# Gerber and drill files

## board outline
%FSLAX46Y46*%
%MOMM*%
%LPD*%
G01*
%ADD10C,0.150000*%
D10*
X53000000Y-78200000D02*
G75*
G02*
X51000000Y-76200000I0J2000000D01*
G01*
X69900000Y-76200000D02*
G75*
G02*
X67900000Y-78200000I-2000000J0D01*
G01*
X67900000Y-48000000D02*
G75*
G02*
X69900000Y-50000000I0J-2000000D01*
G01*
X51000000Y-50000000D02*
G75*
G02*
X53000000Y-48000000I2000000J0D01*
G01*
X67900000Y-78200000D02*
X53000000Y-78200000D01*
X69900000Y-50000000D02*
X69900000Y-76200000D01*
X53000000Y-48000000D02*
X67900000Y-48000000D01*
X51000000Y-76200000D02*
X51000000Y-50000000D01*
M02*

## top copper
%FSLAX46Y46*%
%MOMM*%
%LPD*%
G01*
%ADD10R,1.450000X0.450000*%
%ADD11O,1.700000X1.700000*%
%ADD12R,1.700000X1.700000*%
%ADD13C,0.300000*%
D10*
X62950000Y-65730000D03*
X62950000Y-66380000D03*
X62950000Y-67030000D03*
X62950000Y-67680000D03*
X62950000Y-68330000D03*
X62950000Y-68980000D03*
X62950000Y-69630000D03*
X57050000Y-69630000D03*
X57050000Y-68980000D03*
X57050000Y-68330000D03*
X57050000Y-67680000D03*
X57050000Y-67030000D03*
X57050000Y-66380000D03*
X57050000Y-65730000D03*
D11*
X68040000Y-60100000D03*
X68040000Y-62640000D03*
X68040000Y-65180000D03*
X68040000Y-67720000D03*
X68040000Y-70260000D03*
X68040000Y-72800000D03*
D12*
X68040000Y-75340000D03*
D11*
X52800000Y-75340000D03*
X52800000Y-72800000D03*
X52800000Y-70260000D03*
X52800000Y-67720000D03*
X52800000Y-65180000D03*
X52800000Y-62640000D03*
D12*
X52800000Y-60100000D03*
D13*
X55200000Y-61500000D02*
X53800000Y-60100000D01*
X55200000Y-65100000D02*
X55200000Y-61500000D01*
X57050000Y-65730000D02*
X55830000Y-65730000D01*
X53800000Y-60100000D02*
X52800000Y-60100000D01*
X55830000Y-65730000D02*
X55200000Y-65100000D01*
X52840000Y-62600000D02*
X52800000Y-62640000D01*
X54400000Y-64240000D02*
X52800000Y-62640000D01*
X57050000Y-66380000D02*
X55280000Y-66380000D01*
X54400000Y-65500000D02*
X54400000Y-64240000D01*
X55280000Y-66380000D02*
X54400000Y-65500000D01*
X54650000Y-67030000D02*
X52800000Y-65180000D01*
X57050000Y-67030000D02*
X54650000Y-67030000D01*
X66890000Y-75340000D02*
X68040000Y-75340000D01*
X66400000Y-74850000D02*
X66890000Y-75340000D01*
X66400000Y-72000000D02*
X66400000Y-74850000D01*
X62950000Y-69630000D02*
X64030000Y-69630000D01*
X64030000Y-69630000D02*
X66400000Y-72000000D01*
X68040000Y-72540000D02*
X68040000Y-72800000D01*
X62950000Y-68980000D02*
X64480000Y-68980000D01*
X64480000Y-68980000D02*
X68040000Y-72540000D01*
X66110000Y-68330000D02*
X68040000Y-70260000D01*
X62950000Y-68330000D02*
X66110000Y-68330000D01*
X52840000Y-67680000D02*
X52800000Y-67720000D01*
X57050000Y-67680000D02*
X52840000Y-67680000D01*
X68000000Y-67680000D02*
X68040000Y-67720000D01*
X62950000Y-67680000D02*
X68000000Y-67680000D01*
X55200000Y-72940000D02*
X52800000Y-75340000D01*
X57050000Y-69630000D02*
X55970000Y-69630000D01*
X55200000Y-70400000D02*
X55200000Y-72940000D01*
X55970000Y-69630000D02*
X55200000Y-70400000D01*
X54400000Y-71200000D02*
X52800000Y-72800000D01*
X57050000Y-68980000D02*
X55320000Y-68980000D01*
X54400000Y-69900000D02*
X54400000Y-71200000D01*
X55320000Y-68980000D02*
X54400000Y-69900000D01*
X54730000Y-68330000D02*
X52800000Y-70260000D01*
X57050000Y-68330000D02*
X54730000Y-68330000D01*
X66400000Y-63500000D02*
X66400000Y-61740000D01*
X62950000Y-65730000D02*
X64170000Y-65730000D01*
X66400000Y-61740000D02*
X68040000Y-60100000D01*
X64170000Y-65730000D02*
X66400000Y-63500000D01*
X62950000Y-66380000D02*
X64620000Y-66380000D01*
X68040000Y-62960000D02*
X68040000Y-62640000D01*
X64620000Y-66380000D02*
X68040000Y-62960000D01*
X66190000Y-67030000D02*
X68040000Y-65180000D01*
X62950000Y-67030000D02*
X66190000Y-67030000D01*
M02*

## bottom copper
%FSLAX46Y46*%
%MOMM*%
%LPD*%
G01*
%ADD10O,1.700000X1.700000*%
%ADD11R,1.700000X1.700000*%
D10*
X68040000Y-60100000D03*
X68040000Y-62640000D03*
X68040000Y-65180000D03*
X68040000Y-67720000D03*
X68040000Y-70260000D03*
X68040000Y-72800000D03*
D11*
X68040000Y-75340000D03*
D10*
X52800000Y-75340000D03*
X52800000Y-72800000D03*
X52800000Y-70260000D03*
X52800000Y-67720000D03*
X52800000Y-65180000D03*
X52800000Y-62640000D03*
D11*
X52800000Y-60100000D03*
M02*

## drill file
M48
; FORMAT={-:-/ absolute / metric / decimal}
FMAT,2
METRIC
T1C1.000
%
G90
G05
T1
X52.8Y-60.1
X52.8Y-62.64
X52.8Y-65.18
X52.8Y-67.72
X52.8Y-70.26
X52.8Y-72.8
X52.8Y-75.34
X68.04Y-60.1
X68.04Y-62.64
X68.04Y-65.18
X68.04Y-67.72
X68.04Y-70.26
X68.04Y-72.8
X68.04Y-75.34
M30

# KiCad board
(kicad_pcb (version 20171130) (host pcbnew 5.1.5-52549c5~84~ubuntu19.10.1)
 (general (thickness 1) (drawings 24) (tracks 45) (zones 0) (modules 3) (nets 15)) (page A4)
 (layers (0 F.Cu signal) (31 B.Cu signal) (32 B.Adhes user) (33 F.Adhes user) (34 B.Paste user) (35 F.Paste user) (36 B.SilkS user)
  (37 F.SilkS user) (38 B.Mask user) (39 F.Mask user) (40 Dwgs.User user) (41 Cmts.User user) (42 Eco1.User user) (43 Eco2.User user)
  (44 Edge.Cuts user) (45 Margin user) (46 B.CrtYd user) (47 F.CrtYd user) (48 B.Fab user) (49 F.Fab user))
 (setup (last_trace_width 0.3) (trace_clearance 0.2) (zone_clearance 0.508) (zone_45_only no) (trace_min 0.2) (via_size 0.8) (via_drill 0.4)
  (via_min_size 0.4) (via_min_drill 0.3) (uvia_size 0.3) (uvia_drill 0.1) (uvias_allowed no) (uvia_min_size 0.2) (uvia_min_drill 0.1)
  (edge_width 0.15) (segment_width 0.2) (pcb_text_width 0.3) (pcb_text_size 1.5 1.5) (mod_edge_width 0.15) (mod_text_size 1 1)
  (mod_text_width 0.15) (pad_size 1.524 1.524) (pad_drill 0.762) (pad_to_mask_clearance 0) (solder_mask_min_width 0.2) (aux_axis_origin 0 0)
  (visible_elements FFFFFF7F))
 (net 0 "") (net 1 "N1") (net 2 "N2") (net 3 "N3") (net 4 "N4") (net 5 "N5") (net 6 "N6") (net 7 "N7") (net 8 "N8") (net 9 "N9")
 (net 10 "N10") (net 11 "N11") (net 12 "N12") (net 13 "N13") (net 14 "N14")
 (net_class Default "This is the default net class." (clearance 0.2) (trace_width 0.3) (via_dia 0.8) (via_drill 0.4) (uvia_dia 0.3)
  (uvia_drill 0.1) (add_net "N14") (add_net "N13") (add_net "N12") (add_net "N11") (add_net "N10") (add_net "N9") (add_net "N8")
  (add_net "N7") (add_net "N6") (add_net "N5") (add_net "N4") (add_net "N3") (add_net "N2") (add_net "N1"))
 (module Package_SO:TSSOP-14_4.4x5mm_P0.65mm (layer F.Cu) (at 60 67.68)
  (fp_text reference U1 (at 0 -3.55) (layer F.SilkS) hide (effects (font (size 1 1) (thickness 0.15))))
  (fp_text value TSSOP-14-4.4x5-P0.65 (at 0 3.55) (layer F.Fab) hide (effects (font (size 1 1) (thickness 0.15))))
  (pad 14 smd rect (at 2.95 -1.95) (size 1.45 0.45) (layers F.Cu F.Paste F.Mask) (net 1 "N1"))
  (pad 13 smd rect (at 2.95 -1.3) (size 1.45 0.45) (layers F.Cu F.Paste F.Mask) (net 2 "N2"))
  (pad 12 smd rect (at 2.95 -0.65) (size 1.45 0.45) (layers F.Cu F.Paste F.Mask) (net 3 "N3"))
  (pad 11 smd rect (at 2.95 0) (size 1.45 0.45) (layers F.Cu F.Paste F.Mask) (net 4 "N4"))
  (pad 10 smd rect (at 2.95 0.65) (size 1.45 0.45) (layers F.Cu F.Paste F.Mask) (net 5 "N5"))
  (pad 9 smd rect (at 2.95 1.3) (size 1.45 0.45) (layers F.Cu F.Paste F.Mask) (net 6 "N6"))
  (pad 8 smd rect (at 2.95 1.95) (size 1.45 0.45) (layers F.Cu F.Paste F.Mask) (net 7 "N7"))
  (pad 7 smd rect (at -2.95 1.95) (size 1.45 0.45) (layers F.Cu F.Paste F.Mask) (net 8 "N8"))
  (pad 6 smd rect (at -2.95 1.3) (size 1.45 0.45) (layers F.Cu F.Paste F.Mask) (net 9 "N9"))
  (pad 5 smd rect (at -2.95 0.65) (size 1.45 0.45) (layers F.Cu F.Paste F.Mask) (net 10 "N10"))
  (pad 4 smd rect (at -2.95 0) (size 1.45 0.45) (layers F.Cu F.Paste F.Mask) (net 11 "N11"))
  (pad 3 smd rect (at -2.95 -0.65) (size 1.45 0.45) (layers F.Cu F.Paste F.Mask) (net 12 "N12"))
  (pad 2 smd rect (at -2.95 -1.3) (size 1.45 0.45) (layers F.Cu F.Paste F.Mask) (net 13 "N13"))
  (pad 1 smd rect (at -2.95 -1.95) (size 1.45 0.45) (layers F.Cu F.Paste F.Mask) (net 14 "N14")))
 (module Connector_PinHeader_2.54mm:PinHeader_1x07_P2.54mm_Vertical (layer F.Cu) (at 68.04 75.34 180)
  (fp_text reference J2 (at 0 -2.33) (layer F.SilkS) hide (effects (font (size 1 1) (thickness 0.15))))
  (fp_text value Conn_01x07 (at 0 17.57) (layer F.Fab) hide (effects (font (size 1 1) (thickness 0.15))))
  (pad 7 thru_hole oval (at 0 15.24 180) (size 1.7 1.7) (drill 1) (layers *.Cu *.Mask) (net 1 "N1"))
  (pad 6 thru_hole oval (at 0 12.7 180) (size 1.7 1.7) (drill 1) (layers *.Cu *.Mask) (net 2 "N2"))
  (pad 5 thru_hole oval (at 0 10.16 180) (size 1.7 1.7) (drill 1) (layers *.Cu *.Mask) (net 3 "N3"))
  (pad 4 thru_hole oval (at 0 7.62 180) (size 1.7 1.7) (drill 1) (layers *.Cu *.Mask) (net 4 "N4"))
  (pad 3 thru_hole oval (at 0 5.08 180) (size 1.7 1.7) (drill 1) (layers *.Cu *.Mask) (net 5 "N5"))
  (pad 2 thru_hole oval (at 0 2.54 180) (size 1.7 1.7) (drill 1) (layers *.Cu *.Mask) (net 6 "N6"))
  (pad 1 thru_hole rect (at 0 0 180) (size 1.7 1.7) (drill 1) (layers *.Cu *.Mask) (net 7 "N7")))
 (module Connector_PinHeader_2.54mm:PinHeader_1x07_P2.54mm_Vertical (layer F.Cu) (at 52.8 60.1)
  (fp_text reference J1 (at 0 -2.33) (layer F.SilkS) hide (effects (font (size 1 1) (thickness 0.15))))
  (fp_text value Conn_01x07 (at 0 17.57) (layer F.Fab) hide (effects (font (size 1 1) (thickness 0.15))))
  (pad 7 thru_hole oval (at 0 15.24) (size 1.7 1.7) (drill 1) (layers *.Cu *.Mask) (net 8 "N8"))
  (pad 6 thru_hole oval (at 0 12.7) (size 1.7 1.7) (drill 1) (layers *.Cu *.Mask) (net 9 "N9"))
  (pad 5 thru_hole oval (at 0 10.16) (size 1.7 1.7) (drill 1) (layers *.Cu *.Mask) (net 10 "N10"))
  (pad 4 thru_hole oval (at 0 7.62) (size 1.7 1.7) (drill 1) (layers *.Cu *.Mask) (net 11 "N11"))
  (pad 3 thru_hole oval (at 0 5.08) (size 1.7 1.7) (drill 1) (layers *.Cu *.Mask) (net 12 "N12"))
  (pad 2 thru_hole oval (at 0 2.54) (size 1.7 1.7) (drill 1) (layers *.Cu *.Mask) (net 13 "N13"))
  (pad 1 thru_hole rect (at 0 0) (size 1.7 1.7) (drill 1) (layers *.Cu *.Mask) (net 14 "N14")))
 (gr_arc (start 53 76.2) (end 51 76.2) (angle -90) (layer Edge.Cuts) (width 0.15))
 (gr_arc (start 67.9 76.2) (end 67.9 78.2) (angle -90) (layer Edge.Cuts) (width 0.15))
 (gr_arc (start 67.9 50) (end 69.9 50) (angle -90) (layer Edge.Cuts) (width 0.15))
 (gr_arc (start 53 50) (end 53 48) (angle -90) (layer Edge.Cuts) (width 0.15))
 (gr_line (start 67.9 78.2) (end 53 78.2) (layer Edge.Cuts) (width 0.15))
 (gr_line (start 69.9 50) (end 69.9 76.2) (layer Edge.Cuts) (width 0.15))
 (gr_line (start 53 48) (end 67.9 48) (layer Edge.Cuts) (width 0.15))
 (gr_line (start 51 76.2) (end 51 50) (layer Edge.Cuts) (width 0.15))
 (segment (start 55.2 61.5) (end 53.8 60.1) (width 0.3) (layer F.Cu) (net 14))
 (segment (start 55.2 65.1) (end 55.2 61.5) (width 0.3) (layer F.Cu) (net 14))
 (segment (start 57.05 65.73) (end 55.83 65.73) (width 0.3) (layer F.Cu) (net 14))
 (segment (start 53.8 60.1) (end 52.8 60.1) (width 0.3) (layer F.Cu) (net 14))
 (segment (start 55.83 65.73) (end 55.2 65.1) (width 0.3) (layer F.Cu) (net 14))
 (segment (start 52.84 62.6) (end 52.8 62.64) (width 0.3) (layer F.Cu) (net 13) (status 30))
 (segment (start 54.4 64.24) (end 52.8 62.64) (width 0.3) (layer F.Cu) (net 13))
 (segment (start 57.05 66.38) (end 55.28 66.38) (width 0.3) (layer F.Cu) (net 13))
 (segment (start 54.4 65.5) (end 54.4 64.24) (width 0.3) (layer F.Cu) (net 13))
 (segment (start 55.28 66.38) (end 54.4 65.5) (width 0.3) (layer F.Cu) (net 13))
 (segment (start 54.65 67.03) (end 52.8 65.18) (width 0.3) (layer F.Cu) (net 12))
 (segment (start 57.05 67.03) (end 54.65 67.03) (width 0.3) (layer F.Cu) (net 12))
 (segment (start 66.89 75.34) (end 68.04 75.34) (width 0.3) (layer F.Cu) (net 7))
 (segment (start 66.4 74.85) (end 66.89 75.34) (width 0.3) (layer F.Cu) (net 7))
 (segment (start 66.4 72) (end 66.4 74.85) (width 0.3) (layer F.Cu) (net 7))
 (segment (start 62.95 69.63) (end 64.03 69.63) (width 0.3) (layer F.Cu) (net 7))
 (segment (start 64.03 69.63) (end 66.4 72) (width 0.3) (layer F.Cu) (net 7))
 (segment (start 68.04 72.54) (end 68.04 72.8) (width 0.3) (layer F.Cu) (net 6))
 (segment (start 62.95 68.98) (end 64.48 68.98) (width 0.3) (layer F.Cu) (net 6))
 (segment (start 64.48 68.98) (end 68.04 72.54) (width 0.3) (layer F.Cu) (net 6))
 (segment (start 66.11 68.33) (end 68.04 70.26) (width 0.3) (layer F.Cu) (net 5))
 (segment (start 62.95 68.33) (end 66.11 68.33) (width 0.3) (layer F.Cu) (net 5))
 (segment (start 52.84 67.68) (end 52.8 67.72) (width 0.3) (layer F.Cu) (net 11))
 (segment (start 57.05 67.68) (end 52.84 67.68) (width 0.3) (layer F.Cu) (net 11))
 (segment (start 68 67.68) (end 68.04 67.72) (width 0.3) (layer F.Cu) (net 4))
 (segment (start 62.95 67.68) (end 68 67.68) (width 0.3) (layer F.Cu) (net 4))
 (segment (start 55.2 72.94) (end 52.8 75.34) (width 0.3) (layer F.Cu) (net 8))
 (segment (start 57.05 69.63) (end 55.97 69.63) (width 0.3) (layer F.Cu) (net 8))
 (segment (start 55.2 70.4) (end 55.2 72.94) (width 0.3) (layer F.Cu) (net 8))
 (segment (start 55.97 69.63) (end 55.2 70.4) (width 0.3) (layer F.Cu) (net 8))
 (segment (start 54.4 71.2) (end 52.8 72.8) (width 0.3) (layer F.Cu) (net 9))
 (segment (start 57.05 68.98) (end 55.32 68.98) (width 0.3) (layer F.Cu) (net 9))
 (segment (start 54.4 69.9) (end 54.4 71.2) (width 0.3) (layer F.Cu) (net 9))
 (segment (start 55.32 68.98) (end 54.4 69.9) (width 0.3) (layer F.Cu) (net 9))
 (segment (start 54.73 68.33) (end 52.8 70.26) (width 0.3) (layer F.Cu) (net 10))
 (segment (start 57.05 68.33) (end 54.73 68.33) (width 0.3) (layer F.Cu) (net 10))
 (segment (start 66.4 63.5) (end 66.4 61.74) (width 0.3) (layer F.Cu) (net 1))
 (segment (start 62.95 65.73) (end 64.17 65.73) (width 0.3) (layer F.Cu) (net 1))
 (segment (start 66.4 61.74) (end 68.04 60.1) (width 0.3) (layer F.Cu) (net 1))
 (segment (start 64.17 65.73) (end 66.4 63.5) (width 0.3) (layer F.Cu) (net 1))
 (segment (start 62.95 66.38) (end 64.62 66.38) (width 0.3) (layer F.Cu) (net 2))
 (segment (start 68.04 62.96) (end 68.04 62.64) (width 0.3) (layer F.Cu) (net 2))
 (segment (start 64.62 66.38) (end 68.04 62.96) (width 0.3) (layer F.Cu) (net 2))
 (segment (start 66.19 67.03) (end 68.04 65.18) (width 0.3) (layer F.Cu) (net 3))
 (segment (start 62.95 67.03) (end 66.19 67.03) (width 0.3) (layer F.Cu) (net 3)))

